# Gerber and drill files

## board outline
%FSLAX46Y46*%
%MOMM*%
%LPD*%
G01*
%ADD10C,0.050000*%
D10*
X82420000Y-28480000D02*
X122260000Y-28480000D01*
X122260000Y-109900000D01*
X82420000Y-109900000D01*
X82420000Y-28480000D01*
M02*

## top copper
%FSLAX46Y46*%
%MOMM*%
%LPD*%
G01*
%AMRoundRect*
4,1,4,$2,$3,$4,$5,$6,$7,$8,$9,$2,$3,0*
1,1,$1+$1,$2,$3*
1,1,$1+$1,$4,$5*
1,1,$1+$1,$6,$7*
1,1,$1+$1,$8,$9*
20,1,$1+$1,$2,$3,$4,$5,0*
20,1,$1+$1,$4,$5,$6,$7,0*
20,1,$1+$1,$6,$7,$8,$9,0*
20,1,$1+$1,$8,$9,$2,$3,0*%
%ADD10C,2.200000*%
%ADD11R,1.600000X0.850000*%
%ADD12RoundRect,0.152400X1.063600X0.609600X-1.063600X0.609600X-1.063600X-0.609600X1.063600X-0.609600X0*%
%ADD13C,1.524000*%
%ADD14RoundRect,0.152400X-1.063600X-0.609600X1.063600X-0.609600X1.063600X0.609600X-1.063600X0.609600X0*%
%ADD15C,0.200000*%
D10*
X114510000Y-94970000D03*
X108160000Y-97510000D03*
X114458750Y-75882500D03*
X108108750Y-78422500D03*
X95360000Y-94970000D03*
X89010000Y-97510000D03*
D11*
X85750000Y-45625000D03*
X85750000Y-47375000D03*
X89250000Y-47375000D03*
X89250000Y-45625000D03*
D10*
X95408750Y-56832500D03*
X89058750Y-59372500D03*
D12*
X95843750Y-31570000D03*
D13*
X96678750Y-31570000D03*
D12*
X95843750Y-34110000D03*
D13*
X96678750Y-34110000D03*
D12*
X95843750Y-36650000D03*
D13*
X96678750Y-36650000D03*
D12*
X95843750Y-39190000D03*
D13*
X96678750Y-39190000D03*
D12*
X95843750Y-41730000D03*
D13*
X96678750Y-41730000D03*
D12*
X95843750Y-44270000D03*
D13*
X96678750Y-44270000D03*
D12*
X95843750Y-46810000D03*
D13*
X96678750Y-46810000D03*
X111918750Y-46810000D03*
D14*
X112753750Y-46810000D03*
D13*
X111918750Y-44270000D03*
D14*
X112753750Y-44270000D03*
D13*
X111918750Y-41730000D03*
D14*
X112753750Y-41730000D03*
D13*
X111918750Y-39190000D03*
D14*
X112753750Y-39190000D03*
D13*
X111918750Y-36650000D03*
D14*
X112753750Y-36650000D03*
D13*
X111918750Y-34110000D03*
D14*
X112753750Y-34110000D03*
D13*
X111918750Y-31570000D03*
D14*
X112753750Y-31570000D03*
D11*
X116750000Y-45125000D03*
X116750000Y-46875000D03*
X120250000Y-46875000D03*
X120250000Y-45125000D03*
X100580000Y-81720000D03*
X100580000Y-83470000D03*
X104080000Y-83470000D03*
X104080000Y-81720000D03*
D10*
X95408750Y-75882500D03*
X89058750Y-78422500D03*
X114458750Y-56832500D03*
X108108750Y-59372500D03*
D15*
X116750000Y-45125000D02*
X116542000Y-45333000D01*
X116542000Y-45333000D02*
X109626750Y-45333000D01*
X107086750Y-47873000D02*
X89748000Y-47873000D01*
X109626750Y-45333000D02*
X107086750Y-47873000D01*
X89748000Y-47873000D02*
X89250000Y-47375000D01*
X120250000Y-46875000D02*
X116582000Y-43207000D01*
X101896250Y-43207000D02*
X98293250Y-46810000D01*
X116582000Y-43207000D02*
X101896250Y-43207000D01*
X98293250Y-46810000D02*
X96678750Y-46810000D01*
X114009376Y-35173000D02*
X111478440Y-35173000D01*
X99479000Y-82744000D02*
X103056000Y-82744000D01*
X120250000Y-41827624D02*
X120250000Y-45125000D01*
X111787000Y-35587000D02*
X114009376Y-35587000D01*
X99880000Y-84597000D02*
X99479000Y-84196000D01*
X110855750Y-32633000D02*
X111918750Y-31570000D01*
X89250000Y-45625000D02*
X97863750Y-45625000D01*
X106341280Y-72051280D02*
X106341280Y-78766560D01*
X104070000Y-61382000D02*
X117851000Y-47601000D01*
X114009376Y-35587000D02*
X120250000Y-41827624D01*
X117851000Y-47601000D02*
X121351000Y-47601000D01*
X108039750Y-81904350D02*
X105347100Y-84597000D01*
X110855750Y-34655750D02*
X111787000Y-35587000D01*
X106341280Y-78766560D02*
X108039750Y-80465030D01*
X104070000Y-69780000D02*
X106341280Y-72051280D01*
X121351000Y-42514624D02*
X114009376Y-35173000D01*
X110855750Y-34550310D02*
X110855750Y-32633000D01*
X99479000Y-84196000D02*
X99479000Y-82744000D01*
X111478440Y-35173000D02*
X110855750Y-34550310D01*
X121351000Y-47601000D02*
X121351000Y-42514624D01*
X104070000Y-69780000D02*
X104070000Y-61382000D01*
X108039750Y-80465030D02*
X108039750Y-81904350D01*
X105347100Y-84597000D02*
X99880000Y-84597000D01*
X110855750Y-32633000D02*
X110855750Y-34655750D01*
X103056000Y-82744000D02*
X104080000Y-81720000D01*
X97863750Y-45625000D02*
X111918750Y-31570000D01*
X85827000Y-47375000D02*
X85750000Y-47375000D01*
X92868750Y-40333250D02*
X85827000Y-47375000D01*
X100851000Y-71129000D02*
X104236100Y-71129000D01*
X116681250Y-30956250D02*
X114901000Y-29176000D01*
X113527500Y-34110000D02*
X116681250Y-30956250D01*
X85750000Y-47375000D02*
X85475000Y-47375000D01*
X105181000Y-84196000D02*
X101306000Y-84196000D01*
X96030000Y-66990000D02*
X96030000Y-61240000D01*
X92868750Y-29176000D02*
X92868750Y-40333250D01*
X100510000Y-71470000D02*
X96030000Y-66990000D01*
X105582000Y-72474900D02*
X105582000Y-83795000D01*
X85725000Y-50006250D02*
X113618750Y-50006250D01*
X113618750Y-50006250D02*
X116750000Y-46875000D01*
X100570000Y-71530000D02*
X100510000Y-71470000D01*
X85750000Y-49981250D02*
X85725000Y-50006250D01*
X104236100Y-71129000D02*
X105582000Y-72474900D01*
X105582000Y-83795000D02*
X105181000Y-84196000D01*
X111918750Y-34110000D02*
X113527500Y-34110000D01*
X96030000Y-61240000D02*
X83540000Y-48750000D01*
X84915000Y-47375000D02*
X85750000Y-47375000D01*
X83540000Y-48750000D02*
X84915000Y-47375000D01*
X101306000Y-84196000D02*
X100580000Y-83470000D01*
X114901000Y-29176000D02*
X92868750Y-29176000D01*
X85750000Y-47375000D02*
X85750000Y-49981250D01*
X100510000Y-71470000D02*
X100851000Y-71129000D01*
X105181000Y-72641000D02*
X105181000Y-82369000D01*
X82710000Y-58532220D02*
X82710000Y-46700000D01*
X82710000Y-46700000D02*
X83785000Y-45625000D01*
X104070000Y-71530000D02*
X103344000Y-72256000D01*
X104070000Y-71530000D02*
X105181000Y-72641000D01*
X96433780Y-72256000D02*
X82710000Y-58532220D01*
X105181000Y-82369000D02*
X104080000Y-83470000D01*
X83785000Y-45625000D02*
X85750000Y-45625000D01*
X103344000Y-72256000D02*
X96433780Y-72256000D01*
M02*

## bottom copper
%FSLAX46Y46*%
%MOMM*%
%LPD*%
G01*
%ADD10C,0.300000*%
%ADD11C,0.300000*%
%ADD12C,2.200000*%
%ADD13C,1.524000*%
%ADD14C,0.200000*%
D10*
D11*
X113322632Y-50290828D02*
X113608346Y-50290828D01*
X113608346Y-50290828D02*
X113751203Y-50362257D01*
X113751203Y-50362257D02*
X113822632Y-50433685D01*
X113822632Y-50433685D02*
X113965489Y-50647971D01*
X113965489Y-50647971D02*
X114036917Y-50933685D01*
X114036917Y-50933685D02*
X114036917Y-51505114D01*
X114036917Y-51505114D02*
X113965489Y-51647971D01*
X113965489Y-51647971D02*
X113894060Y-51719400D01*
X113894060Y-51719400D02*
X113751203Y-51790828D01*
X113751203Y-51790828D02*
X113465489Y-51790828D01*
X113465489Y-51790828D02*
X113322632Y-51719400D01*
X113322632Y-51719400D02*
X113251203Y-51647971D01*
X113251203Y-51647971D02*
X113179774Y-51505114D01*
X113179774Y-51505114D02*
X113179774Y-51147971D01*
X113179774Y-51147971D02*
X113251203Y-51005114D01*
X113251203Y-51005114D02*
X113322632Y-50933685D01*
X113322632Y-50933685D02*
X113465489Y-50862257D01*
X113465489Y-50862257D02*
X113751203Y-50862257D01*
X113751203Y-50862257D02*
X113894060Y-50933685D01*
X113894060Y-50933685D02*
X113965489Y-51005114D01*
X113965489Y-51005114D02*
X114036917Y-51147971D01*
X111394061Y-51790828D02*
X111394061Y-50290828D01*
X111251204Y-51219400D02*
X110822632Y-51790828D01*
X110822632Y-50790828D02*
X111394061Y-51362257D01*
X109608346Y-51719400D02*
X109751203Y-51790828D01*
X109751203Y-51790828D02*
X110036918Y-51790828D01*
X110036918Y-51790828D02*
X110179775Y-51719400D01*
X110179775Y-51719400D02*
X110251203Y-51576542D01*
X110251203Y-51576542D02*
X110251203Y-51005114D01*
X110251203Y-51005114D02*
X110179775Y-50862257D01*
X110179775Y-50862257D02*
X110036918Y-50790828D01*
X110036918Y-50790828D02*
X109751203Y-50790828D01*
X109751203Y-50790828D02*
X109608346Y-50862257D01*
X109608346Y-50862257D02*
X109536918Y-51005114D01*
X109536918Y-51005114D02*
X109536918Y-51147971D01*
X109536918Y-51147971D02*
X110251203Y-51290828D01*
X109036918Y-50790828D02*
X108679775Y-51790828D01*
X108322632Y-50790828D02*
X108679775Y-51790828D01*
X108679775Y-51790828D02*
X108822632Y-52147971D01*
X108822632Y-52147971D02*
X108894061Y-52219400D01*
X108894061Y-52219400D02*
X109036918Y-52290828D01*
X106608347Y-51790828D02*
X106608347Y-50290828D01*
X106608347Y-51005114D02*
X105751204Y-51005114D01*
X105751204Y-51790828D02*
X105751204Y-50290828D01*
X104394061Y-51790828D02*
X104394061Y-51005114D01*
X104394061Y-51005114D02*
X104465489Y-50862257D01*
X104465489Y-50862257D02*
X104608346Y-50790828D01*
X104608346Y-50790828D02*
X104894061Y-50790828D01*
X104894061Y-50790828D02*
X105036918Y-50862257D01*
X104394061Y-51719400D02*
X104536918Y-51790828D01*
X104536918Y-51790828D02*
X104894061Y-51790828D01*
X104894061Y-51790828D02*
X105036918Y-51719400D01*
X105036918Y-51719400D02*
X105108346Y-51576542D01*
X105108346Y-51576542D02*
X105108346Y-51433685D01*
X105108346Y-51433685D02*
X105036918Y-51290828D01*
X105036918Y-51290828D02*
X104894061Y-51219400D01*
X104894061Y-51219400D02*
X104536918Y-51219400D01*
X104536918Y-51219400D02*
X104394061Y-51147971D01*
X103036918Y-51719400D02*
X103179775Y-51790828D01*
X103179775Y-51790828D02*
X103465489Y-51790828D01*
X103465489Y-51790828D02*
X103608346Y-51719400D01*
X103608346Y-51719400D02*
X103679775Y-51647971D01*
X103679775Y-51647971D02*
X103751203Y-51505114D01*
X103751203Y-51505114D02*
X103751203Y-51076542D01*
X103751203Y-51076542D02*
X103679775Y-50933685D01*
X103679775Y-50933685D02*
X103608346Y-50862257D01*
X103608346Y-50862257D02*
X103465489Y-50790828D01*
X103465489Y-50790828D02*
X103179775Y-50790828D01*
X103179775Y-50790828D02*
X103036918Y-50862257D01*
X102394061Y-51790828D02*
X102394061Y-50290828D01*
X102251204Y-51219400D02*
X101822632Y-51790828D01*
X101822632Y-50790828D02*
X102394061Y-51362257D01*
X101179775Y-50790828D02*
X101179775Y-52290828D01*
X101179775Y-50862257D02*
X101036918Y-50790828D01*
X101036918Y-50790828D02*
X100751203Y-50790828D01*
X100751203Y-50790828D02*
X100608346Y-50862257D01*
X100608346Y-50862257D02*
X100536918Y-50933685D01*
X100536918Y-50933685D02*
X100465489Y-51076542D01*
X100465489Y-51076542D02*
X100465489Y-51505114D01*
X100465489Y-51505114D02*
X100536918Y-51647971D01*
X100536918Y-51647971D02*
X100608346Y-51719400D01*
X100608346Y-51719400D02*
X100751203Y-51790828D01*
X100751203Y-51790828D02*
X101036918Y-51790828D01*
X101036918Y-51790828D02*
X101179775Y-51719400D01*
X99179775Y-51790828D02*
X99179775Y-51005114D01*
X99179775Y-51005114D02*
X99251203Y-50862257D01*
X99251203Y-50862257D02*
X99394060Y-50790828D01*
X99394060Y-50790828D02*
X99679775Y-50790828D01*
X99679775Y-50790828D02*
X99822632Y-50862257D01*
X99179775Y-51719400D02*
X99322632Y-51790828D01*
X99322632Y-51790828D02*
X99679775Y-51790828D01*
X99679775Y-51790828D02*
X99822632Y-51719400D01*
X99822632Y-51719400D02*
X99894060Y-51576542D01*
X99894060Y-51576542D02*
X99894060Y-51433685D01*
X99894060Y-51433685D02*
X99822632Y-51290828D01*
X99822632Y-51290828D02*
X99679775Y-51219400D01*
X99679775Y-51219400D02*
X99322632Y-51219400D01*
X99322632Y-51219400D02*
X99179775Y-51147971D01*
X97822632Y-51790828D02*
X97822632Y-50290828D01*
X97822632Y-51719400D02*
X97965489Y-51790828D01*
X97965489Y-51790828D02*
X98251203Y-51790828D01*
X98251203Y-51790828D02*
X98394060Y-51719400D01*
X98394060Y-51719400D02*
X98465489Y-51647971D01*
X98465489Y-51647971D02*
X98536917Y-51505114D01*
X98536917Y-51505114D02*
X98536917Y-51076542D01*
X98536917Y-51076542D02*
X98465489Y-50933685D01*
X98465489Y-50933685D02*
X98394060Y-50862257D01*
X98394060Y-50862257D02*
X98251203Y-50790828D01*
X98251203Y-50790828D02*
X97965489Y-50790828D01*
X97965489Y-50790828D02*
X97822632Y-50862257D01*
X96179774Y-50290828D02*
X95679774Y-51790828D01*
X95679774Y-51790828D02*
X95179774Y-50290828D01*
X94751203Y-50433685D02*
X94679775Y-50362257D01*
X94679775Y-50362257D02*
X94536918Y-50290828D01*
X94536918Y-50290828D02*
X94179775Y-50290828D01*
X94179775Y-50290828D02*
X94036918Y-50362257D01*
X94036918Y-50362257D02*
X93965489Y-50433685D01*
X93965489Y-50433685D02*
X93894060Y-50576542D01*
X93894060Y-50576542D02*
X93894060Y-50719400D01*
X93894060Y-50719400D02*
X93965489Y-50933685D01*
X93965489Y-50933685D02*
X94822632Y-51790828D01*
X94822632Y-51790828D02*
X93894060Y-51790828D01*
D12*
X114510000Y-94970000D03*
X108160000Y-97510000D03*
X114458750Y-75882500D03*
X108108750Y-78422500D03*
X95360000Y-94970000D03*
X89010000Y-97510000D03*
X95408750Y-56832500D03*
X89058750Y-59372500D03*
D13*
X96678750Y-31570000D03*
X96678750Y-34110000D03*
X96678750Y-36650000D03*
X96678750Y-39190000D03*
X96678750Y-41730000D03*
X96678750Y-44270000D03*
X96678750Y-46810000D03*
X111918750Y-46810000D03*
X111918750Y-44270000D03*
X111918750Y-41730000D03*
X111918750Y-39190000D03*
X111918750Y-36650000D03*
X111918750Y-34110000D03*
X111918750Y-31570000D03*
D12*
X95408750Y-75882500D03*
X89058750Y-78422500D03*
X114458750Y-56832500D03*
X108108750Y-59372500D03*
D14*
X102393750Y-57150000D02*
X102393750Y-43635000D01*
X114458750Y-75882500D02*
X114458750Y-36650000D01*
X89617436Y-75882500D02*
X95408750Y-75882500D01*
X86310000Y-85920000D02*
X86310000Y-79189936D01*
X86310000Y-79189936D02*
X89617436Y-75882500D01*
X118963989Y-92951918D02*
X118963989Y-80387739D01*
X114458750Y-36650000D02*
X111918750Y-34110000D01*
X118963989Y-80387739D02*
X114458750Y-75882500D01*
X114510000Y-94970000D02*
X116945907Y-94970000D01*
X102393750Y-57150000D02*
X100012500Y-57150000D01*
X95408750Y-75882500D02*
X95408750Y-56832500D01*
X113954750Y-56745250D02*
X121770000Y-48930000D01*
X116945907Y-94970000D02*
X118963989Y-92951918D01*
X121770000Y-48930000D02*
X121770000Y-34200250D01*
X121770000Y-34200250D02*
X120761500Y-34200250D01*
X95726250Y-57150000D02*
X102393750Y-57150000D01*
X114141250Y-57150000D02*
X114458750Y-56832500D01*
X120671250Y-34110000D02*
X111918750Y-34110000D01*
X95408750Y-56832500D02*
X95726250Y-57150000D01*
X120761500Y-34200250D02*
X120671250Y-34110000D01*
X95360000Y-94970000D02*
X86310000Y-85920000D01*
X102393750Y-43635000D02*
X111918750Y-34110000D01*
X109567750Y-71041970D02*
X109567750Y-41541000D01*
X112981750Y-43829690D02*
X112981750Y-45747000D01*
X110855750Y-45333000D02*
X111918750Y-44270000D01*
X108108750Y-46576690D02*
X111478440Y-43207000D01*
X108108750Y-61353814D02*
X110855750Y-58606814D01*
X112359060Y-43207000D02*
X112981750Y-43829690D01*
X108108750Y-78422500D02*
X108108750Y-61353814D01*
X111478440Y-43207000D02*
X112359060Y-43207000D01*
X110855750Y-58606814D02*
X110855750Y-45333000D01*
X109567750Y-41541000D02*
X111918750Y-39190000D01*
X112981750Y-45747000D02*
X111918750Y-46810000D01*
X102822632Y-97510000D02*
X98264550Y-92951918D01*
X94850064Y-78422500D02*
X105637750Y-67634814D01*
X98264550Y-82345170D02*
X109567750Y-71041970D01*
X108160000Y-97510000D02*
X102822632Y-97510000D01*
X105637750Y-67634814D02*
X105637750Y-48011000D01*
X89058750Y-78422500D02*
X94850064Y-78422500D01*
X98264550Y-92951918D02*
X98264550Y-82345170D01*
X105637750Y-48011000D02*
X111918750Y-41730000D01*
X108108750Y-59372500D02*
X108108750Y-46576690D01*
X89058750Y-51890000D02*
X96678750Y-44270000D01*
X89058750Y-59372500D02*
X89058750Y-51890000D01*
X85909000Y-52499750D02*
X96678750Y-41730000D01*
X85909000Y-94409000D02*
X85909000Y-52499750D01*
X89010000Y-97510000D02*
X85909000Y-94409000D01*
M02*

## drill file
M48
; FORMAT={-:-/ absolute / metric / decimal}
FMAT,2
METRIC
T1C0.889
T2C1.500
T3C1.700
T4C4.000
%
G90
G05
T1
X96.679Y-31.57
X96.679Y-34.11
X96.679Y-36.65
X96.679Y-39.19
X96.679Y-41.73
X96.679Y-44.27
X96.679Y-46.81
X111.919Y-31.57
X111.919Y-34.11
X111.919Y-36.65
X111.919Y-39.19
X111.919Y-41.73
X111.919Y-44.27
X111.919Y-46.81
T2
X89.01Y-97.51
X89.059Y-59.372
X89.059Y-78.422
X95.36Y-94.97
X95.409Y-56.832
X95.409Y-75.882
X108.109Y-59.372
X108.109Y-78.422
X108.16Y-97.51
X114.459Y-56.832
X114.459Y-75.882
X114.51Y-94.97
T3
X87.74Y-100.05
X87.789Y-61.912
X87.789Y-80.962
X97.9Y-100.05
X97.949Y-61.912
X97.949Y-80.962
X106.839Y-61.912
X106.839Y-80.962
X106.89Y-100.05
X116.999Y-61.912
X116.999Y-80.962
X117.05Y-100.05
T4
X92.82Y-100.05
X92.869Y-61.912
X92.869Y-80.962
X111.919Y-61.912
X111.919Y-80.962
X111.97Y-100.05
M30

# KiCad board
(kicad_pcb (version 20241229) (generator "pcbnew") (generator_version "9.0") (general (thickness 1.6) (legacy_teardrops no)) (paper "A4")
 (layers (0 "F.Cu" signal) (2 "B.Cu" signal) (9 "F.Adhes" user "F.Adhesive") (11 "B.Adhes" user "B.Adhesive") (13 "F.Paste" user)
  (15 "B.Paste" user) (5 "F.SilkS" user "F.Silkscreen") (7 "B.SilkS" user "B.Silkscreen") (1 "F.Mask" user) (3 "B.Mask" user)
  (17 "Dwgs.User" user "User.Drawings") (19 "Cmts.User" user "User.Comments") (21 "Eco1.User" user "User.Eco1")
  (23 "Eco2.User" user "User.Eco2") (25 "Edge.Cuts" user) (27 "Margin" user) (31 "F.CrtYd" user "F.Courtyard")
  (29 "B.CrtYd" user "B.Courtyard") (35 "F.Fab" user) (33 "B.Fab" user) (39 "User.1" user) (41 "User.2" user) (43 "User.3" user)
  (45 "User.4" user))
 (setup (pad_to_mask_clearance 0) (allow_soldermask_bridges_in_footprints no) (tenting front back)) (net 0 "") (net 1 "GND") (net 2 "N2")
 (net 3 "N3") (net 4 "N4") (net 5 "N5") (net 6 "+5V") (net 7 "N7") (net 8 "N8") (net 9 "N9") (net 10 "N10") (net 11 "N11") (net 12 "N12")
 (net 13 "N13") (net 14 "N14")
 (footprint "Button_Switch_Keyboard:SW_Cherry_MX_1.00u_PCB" (layer "F.Cu") (at 114.51 94.97)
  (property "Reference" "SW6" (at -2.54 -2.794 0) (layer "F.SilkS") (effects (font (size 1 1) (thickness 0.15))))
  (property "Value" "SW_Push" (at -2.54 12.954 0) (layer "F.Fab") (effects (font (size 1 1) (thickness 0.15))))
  (pad "" np_thru_hole circle (at -7.62 5.08) (size 1.7 1.7) (drill 1.7) (layers "*.Cu" "*.Mask"))
  (pad "" np_thru_hole circle (at -2.54 5.08) (size 4 4) (drill 4) (layers "*.Cu" "*.Mask"))
  (pad "" np_thru_hole circle (at 2.54 5.08) (size 1.7 1.7) (drill 1.7) (layers "*.Cu" "*.Mask"))
  (pad "1" thru_hole circle (at 0 0) (size 2.2 2.2) (drill 1.5) (layers "*.Cu" "*.Mask") (remove_unused_layers no) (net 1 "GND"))
  (pad "2" thru_hole circle (at -6.35 2.54) (size 2.2 2.2) (drill 1.5) (layers "*.Cu" "*.Mask") (remove_unused_layers no) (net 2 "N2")))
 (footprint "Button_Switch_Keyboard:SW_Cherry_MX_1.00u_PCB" (layer "F.Cu") (at 114.45875 75.8825)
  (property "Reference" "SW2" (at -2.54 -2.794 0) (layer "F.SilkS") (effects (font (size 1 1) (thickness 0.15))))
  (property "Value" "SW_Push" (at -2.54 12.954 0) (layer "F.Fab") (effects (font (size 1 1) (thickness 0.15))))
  (pad "" np_thru_hole circle (at -7.62 5.08) (size 1.7 1.7) (drill 1.7) (layers "*.Cu" "*.Mask"))
  (pad "" np_thru_hole circle (at -2.54 5.08) (size 4 4) (drill 4) (layers "*.Cu" "*.Mask"))
  (pad "" np_thru_hole circle (at 2.54 5.08) (size 1.7 1.7) (drill 1.7) (layers "*.Cu" "*.Mask"))
  (pad "1" thru_hole circle (at 0 0) (size 2.2 2.2) (drill 1.5) (layers "*.Cu" "*.Mask") (remove_unused_layers no) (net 1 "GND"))
  (pad "2" thru_hole circle (at -6.35 2.54) (size 2.2 2.2) (drill 1.5) (layers "*.Cu" "*.Mask") (remove_unused_layers no) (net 2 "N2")))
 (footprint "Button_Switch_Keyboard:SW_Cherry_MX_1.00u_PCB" (layer "F.Cu") (at 95.36 94.97)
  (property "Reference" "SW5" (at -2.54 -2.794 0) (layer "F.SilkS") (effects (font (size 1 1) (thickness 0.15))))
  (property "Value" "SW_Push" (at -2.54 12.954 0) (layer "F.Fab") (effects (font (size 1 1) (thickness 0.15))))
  (pad "" np_thru_hole circle (at -7.62 5.08) (size 1.7 1.7) (drill 1.7) (layers "*.Cu" "*.Mask"))
  (pad "" np_thru_hole circle (at -2.54 5.08) (size 4 4) (drill 4) (layers "*.Cu" "*.Mask"))
  (pad "" np_thru_hole circle (at 2.54 5.08) (size 1.7 1.7) (drill 1.7) (layers "*.Cu" "*.Mask"))
  (pad "1" thru_hole circle (at 0 0) (size 2.2 2.2) (drill 1.5) (layers "*.Cu" "*.Mask") (remove_unused_layers no) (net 1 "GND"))
  (pad "2" thru_hole circle (at -6.35 2.54) (size 2.2 2.2) (drill 1.5) (layers "*.Cu" "*.Mask") (remove_unused_layers no) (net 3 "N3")))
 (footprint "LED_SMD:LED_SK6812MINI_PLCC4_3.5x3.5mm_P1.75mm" (layer "F.Cu") (at 87.5 46.5)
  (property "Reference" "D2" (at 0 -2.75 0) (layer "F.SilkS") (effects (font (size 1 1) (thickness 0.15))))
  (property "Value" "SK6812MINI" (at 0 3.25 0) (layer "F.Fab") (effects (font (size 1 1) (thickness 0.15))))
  (pad "1" smd rect (at -1.75 -0.875) (size 1.6 0.85) (layers "F.Cu" "F.Mask" "F.Paste") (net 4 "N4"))
  (pad "2" smd rect (at -1.75 0.875) (size 1.6 0.85) (layers "F.Cu" "F.Mask" "F.Paste") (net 1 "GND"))
  (pad "3" smd rect (at 1.75 0.875) (size 1.6 0.85) (layers "F.Cu" "F.Mask" "F.Paste") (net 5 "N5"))
  (pad "4" smd rect (at 1.75 -0.875) (size 1.6 0.85) (layers "F.Cu" "F.Mask" "F.Paste") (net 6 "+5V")))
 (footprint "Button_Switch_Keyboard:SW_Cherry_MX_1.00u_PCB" (layer "F.Cu") (at 95.40875 56.8325)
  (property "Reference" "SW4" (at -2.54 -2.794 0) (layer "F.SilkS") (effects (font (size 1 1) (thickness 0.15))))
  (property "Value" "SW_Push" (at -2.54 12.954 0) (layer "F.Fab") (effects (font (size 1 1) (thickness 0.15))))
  (pad "" np_thru_hole circle (at -7.62 5.08) (size 1.7 1.7) (drill 1.7) (layers "*.Cu" "*.Mask"))
  (pad "" np_thru_hole circle (at -2.54 5.08) (size 4 4) (drill 4) (layers "*.Cu" "*.Mask"))
  (pad "" np_thru_hole circle (at 2.54 5.08) (size 1.7 1.7) (drill 1.7) (layers "*.Cu" "*.Mask"))
  (pad "1" thru_hole circle (at 0 0) (size 2.2 2.2) (drill 1.5) (layers "*.Cu" "*.Mask") (remove_unused_layers no) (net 1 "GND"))
  (pad "2" thru_hole circle (at -6.35 2.54) (size 2.2 2.2) (drill 1.5) (layers "*.Cu" "*.Mask") (remove_unused_layers no) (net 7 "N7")))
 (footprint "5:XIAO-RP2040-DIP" (layer "F.Cu") (at 104.29875 39.19)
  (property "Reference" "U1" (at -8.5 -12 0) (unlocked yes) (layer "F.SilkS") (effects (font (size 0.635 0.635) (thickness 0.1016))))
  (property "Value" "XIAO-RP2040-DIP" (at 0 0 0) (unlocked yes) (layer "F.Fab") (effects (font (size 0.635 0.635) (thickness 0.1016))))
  (pad "1" smd roundrect (at -8.455 -7.62 180) (size 2.432 1.524) (layers "F.Cu" "F.Mask") (roundrect_rratio 0.1) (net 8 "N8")
   (thermal_bridge_angle 45))
  (pad "1" thru_hole circle (at -7.62 -7.62 180) (size 1.524 1.524) (drill 0.889) (layers "*.Cu" "*.Mask") (remove_unused_layers no)
   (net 8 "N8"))
  (pad "2" smd roundrect (at -8.455 -5.08 180) (size 2.432 1.524) (layers "F.Cu" "F.Mask") (roundrect_rratio 0.1) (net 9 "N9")
   (thermal_bridge_angle 45))
  (pad "2" thru_hole circle (at -7.62 -5.08 180) (size 1.524 1.524) (drill 0.889) (layers "*.Cu" "*.Mask") (remove_unused_layers no)
   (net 9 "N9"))
  (pad "3" smd roundrect (at -8.455 -2.54 180) (size 2.432 1.524) (layers "F.Cu" "F.Mask") (roundrect_rratio 0.1) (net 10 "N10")
   (thermal_bridge_angle 45))
  (pad "3" thru_hole circle (at -7.62 -2.54 180) (size 1.524 1.524) (drill 0.889) (layers "*.Cu" "*.Mask") (remove_unused_layers no)
   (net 10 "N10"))
  (pad "4" smd roundrect (at -8.455 0 180) (size 2.432 1.524) (layers "F.Cu" "F.Mask") (roundrect_rratio 0.1) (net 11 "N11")
   (thermal_bridge_angle 45))
  (pad "4" thru_hole circle (at -7.62 0 180) (size 1.524 1.524) (drill 0.889) (layers "*.Cu" "*.Mask") (remove_unused_layers no)
   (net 11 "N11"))
  (pad "5" smd roundrect (at -8.455 2.54 180) (size 2.432 1.524) (layers "F.Cu" "F.Mask") (roundrect_rratio 0.1) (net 3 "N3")
   (thermal_bridge_angle 45))
  (pad "5" thru_hole circle (at -7.62 2.54 180) (size 1.524 1.524) (drill 0.889) (layers "*.Cu" "*.Mask") (remove_unused_layers no)
   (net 3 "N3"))
  (pad "6" smd roundrect (at -8.455 5.08 180) (size 2.432 1.524) (layers "F.Cu" "F.Mask") (roundrect_rratio 0.1) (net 7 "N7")
   (thermal_bridge_angle 45))
  (pad "6" thru_hole circle (at -7.62 5.08 180) (size 1.524 1.524) (drill 0.889) (layers "*.Cu" "*.Mask") (remove_unused_layers no)
   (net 7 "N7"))
  (pad "7" smd roundrect (at -8.455 7.62 180) (size 2.432 1.524) (layers "F.Cu" "F.Mask") (roundrect_rratio 0.1) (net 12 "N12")
   (thermal_bridge_angle 45))
  (pad "7" thru_hole circle (at -7.62 7.62 180) (size 1.524 1.524) (drill 0.889) (layers "*.Cu" "*.Mask") (remove_unused_layers no)
   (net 12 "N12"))
  (pad "8" thru_hole circle (at 7.62 7.62) (size 1.524 1.524) (drill 0.889) (layers "*.Cu" "*.Mask") (remove_unused_layers no) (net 2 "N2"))
  (pad "8" smd roundrect (at 8.455 7.62) (size 2.432 1.524) (layers "F.Cu" "F.Mask") (roundrect_rratio 0.1) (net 2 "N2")
   (thermal_bridge_angle 45))
  (pad "9" thru_hole circle (at 7.62 5.08) (size 1.524 1.524) (drill 0.889) (layers "*.Cu" "*.Mask") (remove_unused_layers no) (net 2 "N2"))
  (pad "9" smd roundrect (at 8.455 5.08) (size 2.432 1.524) (layers "F.Cu" "F.Mask") (roundrect_rratio 0.1) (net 2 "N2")
   (thermal_bridge_angle 45))
  (pad "10" thru_hole circle (at 7.62 2.54) (size 1.524 1.524) (drill 0.889) (layers "*.Cu" "*.Mask") (remove_unused_layers no) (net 2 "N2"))
  (pad "10" smd roundrect (at 8.455 2.54) (size 2.432 1.524) (layers "F.Cu" "F.Mask") (roundrect_rratio 0.1) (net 2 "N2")
   (thermal_bridge_angle 45))
  (pad "11" thru_hole circle (at 7.62 0) (size 1.524 1.524) (drill 0.889) (layers "*.Cu" "*.Mask") (remove_unused_layers no) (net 2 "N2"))
  (pad "11" smd roundrect (at 8.455 0) (size 2.432 1.524) (layers "F.Cu" "F.Mask") (roundrect_rratio 0.1) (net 2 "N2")
   (thermal_bridge_angle 45))
  (pad "12" thru_hole circle (at 7.62 -2.54) (size 1.524 1.524) (drill 0.889) (layers "*.Cu" "*.Mask") (remove_unused_layers no)
   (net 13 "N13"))
  (pad "12" smd roundrect (at 8.455 -2.54) (size 2.432 1.524) (layers "F.Cu" "F.Mask") (roundrect_rratio 0.1) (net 13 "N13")
   (thermal_bridge_angle 45))
  (pad "13" thru_hole circle (at 7.62 -5.08) (size 1.524 1.524) (drill 0.889) (layers "*.Cu" "*.Mask") (remove_unused_layers no)
   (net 1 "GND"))
  (pad "13" smd roundrect (at 8.455 -5.08) (size 2.432 1.524) (layers "F.Cu" "F.Mask") (roundrect_rratio 0.1) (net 1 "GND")
   (thermal_bridge_angle 45))
  (pad "14" thru_hole circle (at 7.62 -7.62) (size 1.524 1.524) (drill 0.889) (layers "*.Cu" "*.Mask") (remove_unused_layers no)
   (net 6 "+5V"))
  (pad "14" smd roundrect (at 8.455 -7.62) (size 2.432 1.524) (layers "F.Cu" "F.Mask") (roundrect_rratio 0.1) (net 6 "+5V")
   (thermal_bridge_angle 45)))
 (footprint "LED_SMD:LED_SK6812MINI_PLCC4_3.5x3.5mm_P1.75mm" (layer "F.Cu") (at 118.5 46)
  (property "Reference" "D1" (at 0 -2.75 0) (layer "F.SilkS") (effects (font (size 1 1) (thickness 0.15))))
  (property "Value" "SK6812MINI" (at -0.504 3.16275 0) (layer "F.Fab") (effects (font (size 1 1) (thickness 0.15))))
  (pad "1" smd rect (at -1.75 -0.875) (size 1.6 0.85) (layers "F.Cu" "F.Mask" "F.Paste") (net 5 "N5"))
  (pad "2" smd rect (at -1.75 0.875) (size 1.6 0.85) (layers "F.Cu" "F.Mask" "F.Paste") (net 1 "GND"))
  (pad "3" smd rect (at 1.75 0.875) (size 1.6 0.85) (layers "F.Cu" "F.Mask" "F.Paste") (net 12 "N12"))
  (pad "4" smd rect (at 1.75 -0.875) (size 1.6 0.85) (layers "F.Cu" "F.Mask" "F.Paste") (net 6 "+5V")))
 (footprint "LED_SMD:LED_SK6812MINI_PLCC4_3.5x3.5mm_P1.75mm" (layer "F.Cu") (at 102.33 82.595)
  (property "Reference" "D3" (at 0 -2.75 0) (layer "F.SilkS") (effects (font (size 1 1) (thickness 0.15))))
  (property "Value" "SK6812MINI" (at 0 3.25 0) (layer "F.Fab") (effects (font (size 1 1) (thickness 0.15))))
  (pad "1" smd rect (at -1.75 -0.875) (size 1.6 0.85) (layers "F.Cu" "F.Mask" "F.Paste") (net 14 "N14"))
  (pad "2" smd rect (at -1.75 0.875) (size 1.6 0.85) (layers "F.Cu" "F.Mask" "F.Paste") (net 1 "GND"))
  (pad "3" smd rect (at 1.75 0.875) (size 1.6 0.85) (layers "F.Cu" "F.Mask" "F.Paste") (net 4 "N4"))
  (pad "4" smd rect (at 1.75 -0.875) (size 1.6 0.85) (layers "F.Cu" "F.Mask" "F.Paste") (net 6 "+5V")))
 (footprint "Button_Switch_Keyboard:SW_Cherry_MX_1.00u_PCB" (layer "F.Cu") (at 95.40875 75.8825)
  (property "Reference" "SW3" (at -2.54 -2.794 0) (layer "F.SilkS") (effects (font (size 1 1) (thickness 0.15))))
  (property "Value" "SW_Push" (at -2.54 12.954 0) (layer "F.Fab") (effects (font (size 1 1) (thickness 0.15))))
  (pad "" np_thru_hole circle (at -7.62 5.08) (size 1.7 1.7) (drill 1.7) (layers "*.Cu" "*.Mask"))
  (pad "" np_thru_hole circle (at -2.54 5.08) (size 4 4) (drill 4) (layers "*.Cu" "*.Mask"))
  (pad "" np_thru_hole circle (at 2.54 5.08) (size 1.7 1.7) (drill 1.7) (layers "*.Cu" "*.Mask"))
  (pad "1" thru_hole circle (at 0 0) (size 2.2 2.2) (drill 1.5) (layers "*.Cu" "*.Mask") (remove_unused_layers no) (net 1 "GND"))
  (pad "2" thru_hole circle (at -6.35 2.54) (size 2.2 2.2) (drill 1.5) (layers "*.Cu" "*.Mask") (remove_unused_layers no) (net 2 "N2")))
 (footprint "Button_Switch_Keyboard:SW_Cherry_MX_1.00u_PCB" (layer "F.Cu") (at 114.45875 56.8325)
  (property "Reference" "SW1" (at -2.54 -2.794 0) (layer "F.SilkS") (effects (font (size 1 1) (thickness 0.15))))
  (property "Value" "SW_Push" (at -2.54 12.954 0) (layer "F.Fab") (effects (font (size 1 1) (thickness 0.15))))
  (pad "" np_thru_hole circle (at -7.62 5.08) (size 1.7 1.7) (drill 1.7) (layers "*.Cu" "*.Mask"))
  (pad "" np_thru_hole circle (at -2.54 5.08) (size 4 4) (drill 4) (layers "*.Cu" "*.Mask"))
  (pad "" np_thru_hole circle (at 2.54 5.08) (size 1.7 1.7) (drill 1.7) (layers "*.Cu" "*.Mask"))
  (pad "1" thru_hole circle (at 0 0) (size 2.2 2.2) (drill 1.5) (layers "*.Cu" "*.Mask") (remove_unused_layers no) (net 1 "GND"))
  (pad "2" thru_hole circle (at -6.35 2.54) (size 2.2 2.2) (drill 1.5) (layers "*.Cu" "*.Mask") (remove_unused_layers no) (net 2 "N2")))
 (gr_rect (start 82.42 28.48) (end 122.26 109.9) (stroke (width 0.05) (type default)) (fill no) (layer "Edge.Cuts"))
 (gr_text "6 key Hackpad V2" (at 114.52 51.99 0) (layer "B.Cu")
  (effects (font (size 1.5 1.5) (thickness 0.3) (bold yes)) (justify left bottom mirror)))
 (segment (start 116.75 45.125) (end 116.542 45.333) (width 0.2) (layer "F.Cu") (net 5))
 (segment (start 116.542 45.333) (end 109.62675 45.333) (width 0.2) (layer "F.Cu") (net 5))
 (segment (start 107.08675 47.873) (end 89.748 47.873) (width 0.2) (layer "F.Cu") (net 5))
 (segment (start 109.62675 45.333) (end 107.08675 47.873) (width 0.2) (layer "F.Cu") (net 5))
 (segment (start 89.748 47.873) (end 89.25 47.375) (width 0.2) (layer "F.Cu") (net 5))
 (segment (start 120.25 46.875) (end 116.582 43.207) (width 0.2) (layer "F.Cu") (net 12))
 (segment (start 101.89625 43.207) (end 98.29325 46.81) (width 0.2) (layer "F.Cu") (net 12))
 (segment (start 116.582 43.207) (end 101.89625 43.207) (width 0.2) (layer "F.Cu") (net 12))
 (segment (start 98.29325 46.81) (end 96.67875 46.81) (width 0.2) (layer "F.Cu") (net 12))
 (segment (start 114.009376 35.173) (end 111.47844 35.173) (width 0.2) (layer "F.Cu") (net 6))
 (segment (start 99.479 82.744) (end 103.056 82.744) (width 0.2) (layer "F.Cu") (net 6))
 (segment (start 120.25 41.827624) (end 120.25 45.125) (width 0.2) (layer "F.Cu") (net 6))
 (segment (start 111.787 35.587) (end 114.009376 35.587) (width 0.2) (layer "F.Cu") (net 6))
 (segment (start 99.88 84.597) (end 99.479 84.196) (width 0.2) (layer "F.Cu") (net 6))
 (segment (start 110.85575 32.633) (end 111.91875 31.57) (width 0.2) (layer "F.Cu") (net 6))
 (segment (start 89.25 45.625) (end 97.86375 45.625) (width 0.2) (layer "F.Cu") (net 6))
 (segment (start 106.34128 72.05128) (end 106.34128 78.76656) (width 0.2) (layer "F.Cu") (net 6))
 (segment (start 104.07 61.382) (end 117.851 47.601) (width 0.2) (layer "F.Cu") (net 6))
 (segment (start 114.009376 35.587) (end 120.25 41.827624) (width 0.2) (layer "F.Cu") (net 6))
 (segment (start 117.851 47.601) (end 121.351 47.601) (width 0.2) (layer "F.Cu") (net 6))
 (segment (start 108.03975 81.90435) (end 105.3471 84.597) (width 0.2) (layer "F.Cu") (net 6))
 (segment (start 110.85575 34.65575) (end 111.787 35.587) (width 0.2) (layer "F.Cu") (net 6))
 (segment (start 106.34128 78.76656) (end 108.03975 80.46503) (width 0.2) (layer "F.Cu") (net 6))
 (segment (start 104.07 69.78) (end 106.34128 72.05128) (width 0.2) (layer "F.Cu") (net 6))
 (segment (start 121.351 42.514624) (end 114.009376 35.173) (width 0.2) (layer "F.Cu") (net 6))
 (segment (start 110.85575 34.55031) (end 110.85575 32.633) (width 0.2) (layer "F.Cu") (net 6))
 (segment (start 99.479 84.196) (end 99.479 82.744) (width 0.2) (layer "F.Cu") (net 6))
 (segment (start 111.47844 35.173) (end 110.85575 34.55031) (width 0.2) (layer "F.Cu") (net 6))
 (segment (start 121.351 47.601) (end 121.351 42.514624) (width 0.2) (layer "F.Cu") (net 6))
 (segment (start 104.07 69.78) (end 104.07 61.382) (width 0.2) (layer "F.Cu") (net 6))
 (segment (start 108.03975 80.46503) (end 108.03975 81.90435) (width 0.2) (layer "F.Cu") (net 6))
 (segment (start 105.3471 84.597) (end 99.88 84.597) (width 0.2) (layer "F.Cu") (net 6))
 (segment (start 110.85575 32.633) (end 110.85575 34.65575) (width 0.2) (layer "F.Cu") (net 6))
 (segment (start 103.056 82.744) (end 104.08 81.72) (width 0.2) (layer "F.Cu") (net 6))
 (segment (start 97.86375 45.625) (end 111.91875 31.57) (width 0.2) (layer "F.Cu") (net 6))
 (segment (start 85.827 47.375) (end 85.75 47.375) (width 0.2) (layer "F.Cu") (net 1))
 (segment (start 92.86875 40.33325) (end 85.827 47.375) (width 0.2) (layer "F.Cu") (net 1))
 (segment (start 100.851 71.129) (end 104.2361 71.129) (width 0.2) (layer "F.Cu") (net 1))
 (segment (start 116.68125 30.95625) (end 114.901 29.176) (width 0.2) (layer "F.Cu") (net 1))
 (segment (start 113.5275 34.11) (end 116.68125 30.95625) (width 0.2) (layer "F.Cu") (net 1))
 (segment (start 85.75 47.375) (end 85.475 47.375) (width 0.2) (layer "F.Cu") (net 1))
 (segment (start 105.181 84.196) (end 101.306 84.196) (width 0.2) (layer "F.Cu") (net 1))
 (segment (start 96.03 66.99) (end 96.03 61.24) (width 0.2) (layer "F.Cu") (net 1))
 (segment (start 92.86875 29.176) (end 92.86875 40.33325) (width 0.2) (layer "F.Cu") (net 1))
 (segment (start 100.51 71.47) (end 96.03 66.99) (width 0.2) (layer "F.Cu") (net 1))
 (segment (start 105.582 72.4749) (end 105.582 83.795) (width 0.2) (layer "F.Cu") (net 1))
 (segment (start 85.725 50.00625) (end 113.61875 50.00625) (width 0.2) (layer "F.Cu") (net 1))
 (segment (start 113.61875 50.00625) (end 116.75 46.875) (width 0.2) (layer "F.Cu") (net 1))
 (segment (start 100.57 71.53) (end 100.51 71.47) (width 0.2) (layer "F.Cu") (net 1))
 (segment (start 85.75 49.98125) (end 85.725 50.00625) (width 0.2) (layer "F.Cu") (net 1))
 (segment (start 104.2361 71.129) (end 105.582 72.4749) (width 0.2) (layer "F.Cu") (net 1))
 (segment (start 105.582 83.795) (end 105.181 84.196) (width 0.2) (layer "F.Cu") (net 1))
 (segment (start 111.91875 34.11) (end 113.5275 34.11) (width 0.2) (layer "F.Cu") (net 1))
 (segment (start 96.03 61.24) (end 83.54 48.75) (width 0.2) (layer "F.Cu") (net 1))
 (segment (start 84.915 47.375) (end 85.75 47.375) (width 0.2) (layer "F.Cu") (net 1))
 (segment (start 83.54 48.75) (end 84.915 47.375) (width 0.2) (layer "F.Cu") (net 1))
 (segment (start 101.306 84.196) (end 100.58 83.47) (width 0.2) (layer "F.Cu") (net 1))
 (segment (start 114.901 29.176) (end 92.86875 29.176) (width 0.2) (layer "F.Cu") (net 1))
 (segment (start 85.75 47.375) (end 85.75 49.98125) (width 0.2) (layer "F.Cu") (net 1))
 (segment (start 100.51 71.47) (end 100.851 71.129) (width 0.2) (layer "F.Cu") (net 1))
 (segment (start 102.39375 57.15) (end 102.39375 43.635) (width 0.2) (layer "B.Cu") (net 1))
 (segment (start 114.45875 75.8825) (end 114.45875 36.65) (width 0.2) (layer "B.Cu") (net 1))
 (segment (start 89.617436 75.8825) (end 95.40875 75.8825) (width 0.2) (layer "B.Cu") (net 1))
 (segment (start 86.31 85.92) (end 86.31 79.189936) (width 0.2) (layer "B.Cu") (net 1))
 (segment (start 86.31 79.189936) (end 89.617436 75.8825) (width 0.2) (layer "B.Cu") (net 1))
 (segment (start 118.963989 92.951918) (end 118.963989 80.387739) (width 0.2) (layer "B.Cu") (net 1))
 (segment (start 114.45875 36.65) (end 111.91875 34.11) (width 0.2) (layer "B.Cu") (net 1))
 (segment (start 118.963989 80.387739) (end 114.45875 75.8825) (width 0.2) (layer "B.Cu") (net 1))
 (segment (start 114.51 94.97) (end 116.945907 94.97) (width 0.2) (layer "B.Cu") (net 1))
 (segment (start 102.39375 57.15) (end 100.0125 57.15) (width 0.2) (layer "B.Cu") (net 1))
 (segment (start 95.40875 75.8825) (end 95.40875 56.8325) (width 0.2) (layer "B.Cu") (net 1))
 (segment (start 113.95475 56.74525) (end 121.77 48.93) (width 0.2) (layer "B.Cu") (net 1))
 (segment (start 116.945907 94.97) (end 118.963989 92.951918) (width 0.2) (layer "B.Cu") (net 1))
 (segment (start 121.77 48.93) (end 121.77 34.20025) (width 0.2) (layer "B.Cu") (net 1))
 (segment (start 121.77 34.20025) (end 120.7615 34.20025) (width 0.2) (layer "B.Cu") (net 1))
 (segment (start 95.72625 57.15) (end 102.39375 57.15) (width 0.2) (layer "B.Cu") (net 1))
 (segment (start 114.14125 57.15) (end 114.45875 56.8325) (width 0.2) (layer "B.Cu") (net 1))
 (segment (start 120.67125 34.11) (end 111.91875 34.11) (width 0.2) (layer "B.Cu") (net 1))
 (segment (start 95.40875 56.8325) (end 95.72625 57.15) (width 0.2) (layer "B.Cu") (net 1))
 (segment (start 120.7615 34.20025) (end 120.67125 34.11) (width 0.2) (layer "B.Cu") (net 1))
 (segment (start 95.36 94.97) (end 86.31 85.92) (width 0.2) (layer "B.Cu") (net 1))
 (segment (start 102.39375 43.635) (end 111.91875 34.11) (width 0.2) (layer "B.Cu") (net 1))
 (segment (start 109.56775 71.04197) (end 109.56775 41.541) (width 0.2) (layer "B.Cu") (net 2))
 (segment (start 112.98175 43.82969) (end 112.98175 45.747) (width 0.2) (layer "B.Cu") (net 2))
 (segment (start 110.85575 45.333) (end 111.91875 44.27) (width 0.2) (layer "B.Cu") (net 2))
 (segment (start 108.10875 46.57669) (end 111.47844 43.207) (width 0.2) (layer "B.Cu") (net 2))
 (segment (start 108.10875 61.353814) (end 110.85575 58.606814) (width 0.2) (layer "B.Cu") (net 2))
 (segment (start 112.35906 43.207) (end 112.98175 43.82969) (width 0.2) (layer "B.Cu") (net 2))
 (segment (start 108.10875 78.4225) (end 108.10875 61.353814) (width 0.2) (layer "B.Cu") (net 2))
 (segment (start 111.47844 43.207) (end 112.35906 43.207) (width 0.2) (layer "B.Cu") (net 2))
 (segment (start 110.85575 58.606814) (end 110.85575 45.333) (width 0.2) (layer "B.Cu") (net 2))
 (segment (start 109.56775 41.541) (end 111.91875 39.19) (width 0.2) (layer "B.Cu") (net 2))
 (segment (start 112.98175 45.747) (end 111.91875 46.81) (width 0.2) (layer "B.Cu") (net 2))
 (segment (start 102.822632 97.51) (end 98.26455 92.951918) (width 0.2) (layer "B.Cu") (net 2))
 (segment (start 94.850064 78.4225) (end 105.63775 67.634814) (width 0.2) (layer "B.Cu") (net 2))
 (segment (start 98.26455 82.34517) (end 109.56775 71.04197) (width 0.2) (layer "B.Cu") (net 2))
 (segment (start 108.16 97.51) (end 102.822632 97.51) (width 0.2) (layer "B.Cu") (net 2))
 (segment (start 105.63775 67.634814) (end 105.63775 48.011) (width 0.2) (layer "B.Cu") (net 2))
 (segment (start 89.05875 78.4225) (end 94.850064 78.4225) (width 0.2) (layer "B.Cu") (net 2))
 (segment (start 98.26455 92.951918) (end 98.26455 82.34517) (width 0.2) (layer "B.Cu") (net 2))
 (segment (start 105.63775 48.011) (end 111.91875 41.73) (width 0.2) (layer "B.Cu") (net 2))
 (segment (start 108.10875 59.3725) (end 108.10875 46.57669) (width 0.2) (layer "B.Cu") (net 2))
 (segment (start 89.05875 51.89) (end 96.67875 44.27) (width 0.2) (layer "B.Cu") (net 7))
 (segment (start 89.05875 59.3725) (end 89.05875 51.89) (width 0.2) (layer "B.Cu") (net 7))
 (segment (start 105.181 72.641) (end 105.181 82.369) (width 0.2) (layer "F.Cu") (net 4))
 (segment (start 82.71 58.53222) (end 82.71 46.7) (width 0.2) (layer "F.Cu") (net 4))
 (segment (start 82.71 46.7) (end 83.785 45.625) (width 0.2) (layer "F.Cu") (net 4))
 (segment (start 104.07 71.53) (end 103.344 72.256) (width 0.2) (layer "F.Cu") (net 4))
 (segment (start 104.07 71.53) (end 105.181 72.641) (width 0.2) (layer "F.Cu") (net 4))
 (segment (start 96.43378 72.256) (end 82.71 58.53222) (width 0.2) (layer "F.Cu") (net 4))
 (segment (start 105.181 82.369) (end 104.08 83.47) (width 0.2) (layer "F.Cu") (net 4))
 (segment (start 83.785 45.625) (end 85.75 45.625) (width 0.2) (layer "F.Cu") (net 4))
 (segment (start 103.344 72.256) (end 96.43378 72.256) (width 0.2) (layer "F.Cu") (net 4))
 (segment (start 85.909 52.49975) (end 96.67875 41.73) (width 0.2) (layer "B.Cu") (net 3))
 (segment (start 85.909 94.409) (end 85.909 52.49975) (width 0.2) (layer "B.Cu") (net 3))
 (segment (start 89.01 97.51) (end 85.909 94.409) (width 0.2) (layer "B.Cu") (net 3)))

